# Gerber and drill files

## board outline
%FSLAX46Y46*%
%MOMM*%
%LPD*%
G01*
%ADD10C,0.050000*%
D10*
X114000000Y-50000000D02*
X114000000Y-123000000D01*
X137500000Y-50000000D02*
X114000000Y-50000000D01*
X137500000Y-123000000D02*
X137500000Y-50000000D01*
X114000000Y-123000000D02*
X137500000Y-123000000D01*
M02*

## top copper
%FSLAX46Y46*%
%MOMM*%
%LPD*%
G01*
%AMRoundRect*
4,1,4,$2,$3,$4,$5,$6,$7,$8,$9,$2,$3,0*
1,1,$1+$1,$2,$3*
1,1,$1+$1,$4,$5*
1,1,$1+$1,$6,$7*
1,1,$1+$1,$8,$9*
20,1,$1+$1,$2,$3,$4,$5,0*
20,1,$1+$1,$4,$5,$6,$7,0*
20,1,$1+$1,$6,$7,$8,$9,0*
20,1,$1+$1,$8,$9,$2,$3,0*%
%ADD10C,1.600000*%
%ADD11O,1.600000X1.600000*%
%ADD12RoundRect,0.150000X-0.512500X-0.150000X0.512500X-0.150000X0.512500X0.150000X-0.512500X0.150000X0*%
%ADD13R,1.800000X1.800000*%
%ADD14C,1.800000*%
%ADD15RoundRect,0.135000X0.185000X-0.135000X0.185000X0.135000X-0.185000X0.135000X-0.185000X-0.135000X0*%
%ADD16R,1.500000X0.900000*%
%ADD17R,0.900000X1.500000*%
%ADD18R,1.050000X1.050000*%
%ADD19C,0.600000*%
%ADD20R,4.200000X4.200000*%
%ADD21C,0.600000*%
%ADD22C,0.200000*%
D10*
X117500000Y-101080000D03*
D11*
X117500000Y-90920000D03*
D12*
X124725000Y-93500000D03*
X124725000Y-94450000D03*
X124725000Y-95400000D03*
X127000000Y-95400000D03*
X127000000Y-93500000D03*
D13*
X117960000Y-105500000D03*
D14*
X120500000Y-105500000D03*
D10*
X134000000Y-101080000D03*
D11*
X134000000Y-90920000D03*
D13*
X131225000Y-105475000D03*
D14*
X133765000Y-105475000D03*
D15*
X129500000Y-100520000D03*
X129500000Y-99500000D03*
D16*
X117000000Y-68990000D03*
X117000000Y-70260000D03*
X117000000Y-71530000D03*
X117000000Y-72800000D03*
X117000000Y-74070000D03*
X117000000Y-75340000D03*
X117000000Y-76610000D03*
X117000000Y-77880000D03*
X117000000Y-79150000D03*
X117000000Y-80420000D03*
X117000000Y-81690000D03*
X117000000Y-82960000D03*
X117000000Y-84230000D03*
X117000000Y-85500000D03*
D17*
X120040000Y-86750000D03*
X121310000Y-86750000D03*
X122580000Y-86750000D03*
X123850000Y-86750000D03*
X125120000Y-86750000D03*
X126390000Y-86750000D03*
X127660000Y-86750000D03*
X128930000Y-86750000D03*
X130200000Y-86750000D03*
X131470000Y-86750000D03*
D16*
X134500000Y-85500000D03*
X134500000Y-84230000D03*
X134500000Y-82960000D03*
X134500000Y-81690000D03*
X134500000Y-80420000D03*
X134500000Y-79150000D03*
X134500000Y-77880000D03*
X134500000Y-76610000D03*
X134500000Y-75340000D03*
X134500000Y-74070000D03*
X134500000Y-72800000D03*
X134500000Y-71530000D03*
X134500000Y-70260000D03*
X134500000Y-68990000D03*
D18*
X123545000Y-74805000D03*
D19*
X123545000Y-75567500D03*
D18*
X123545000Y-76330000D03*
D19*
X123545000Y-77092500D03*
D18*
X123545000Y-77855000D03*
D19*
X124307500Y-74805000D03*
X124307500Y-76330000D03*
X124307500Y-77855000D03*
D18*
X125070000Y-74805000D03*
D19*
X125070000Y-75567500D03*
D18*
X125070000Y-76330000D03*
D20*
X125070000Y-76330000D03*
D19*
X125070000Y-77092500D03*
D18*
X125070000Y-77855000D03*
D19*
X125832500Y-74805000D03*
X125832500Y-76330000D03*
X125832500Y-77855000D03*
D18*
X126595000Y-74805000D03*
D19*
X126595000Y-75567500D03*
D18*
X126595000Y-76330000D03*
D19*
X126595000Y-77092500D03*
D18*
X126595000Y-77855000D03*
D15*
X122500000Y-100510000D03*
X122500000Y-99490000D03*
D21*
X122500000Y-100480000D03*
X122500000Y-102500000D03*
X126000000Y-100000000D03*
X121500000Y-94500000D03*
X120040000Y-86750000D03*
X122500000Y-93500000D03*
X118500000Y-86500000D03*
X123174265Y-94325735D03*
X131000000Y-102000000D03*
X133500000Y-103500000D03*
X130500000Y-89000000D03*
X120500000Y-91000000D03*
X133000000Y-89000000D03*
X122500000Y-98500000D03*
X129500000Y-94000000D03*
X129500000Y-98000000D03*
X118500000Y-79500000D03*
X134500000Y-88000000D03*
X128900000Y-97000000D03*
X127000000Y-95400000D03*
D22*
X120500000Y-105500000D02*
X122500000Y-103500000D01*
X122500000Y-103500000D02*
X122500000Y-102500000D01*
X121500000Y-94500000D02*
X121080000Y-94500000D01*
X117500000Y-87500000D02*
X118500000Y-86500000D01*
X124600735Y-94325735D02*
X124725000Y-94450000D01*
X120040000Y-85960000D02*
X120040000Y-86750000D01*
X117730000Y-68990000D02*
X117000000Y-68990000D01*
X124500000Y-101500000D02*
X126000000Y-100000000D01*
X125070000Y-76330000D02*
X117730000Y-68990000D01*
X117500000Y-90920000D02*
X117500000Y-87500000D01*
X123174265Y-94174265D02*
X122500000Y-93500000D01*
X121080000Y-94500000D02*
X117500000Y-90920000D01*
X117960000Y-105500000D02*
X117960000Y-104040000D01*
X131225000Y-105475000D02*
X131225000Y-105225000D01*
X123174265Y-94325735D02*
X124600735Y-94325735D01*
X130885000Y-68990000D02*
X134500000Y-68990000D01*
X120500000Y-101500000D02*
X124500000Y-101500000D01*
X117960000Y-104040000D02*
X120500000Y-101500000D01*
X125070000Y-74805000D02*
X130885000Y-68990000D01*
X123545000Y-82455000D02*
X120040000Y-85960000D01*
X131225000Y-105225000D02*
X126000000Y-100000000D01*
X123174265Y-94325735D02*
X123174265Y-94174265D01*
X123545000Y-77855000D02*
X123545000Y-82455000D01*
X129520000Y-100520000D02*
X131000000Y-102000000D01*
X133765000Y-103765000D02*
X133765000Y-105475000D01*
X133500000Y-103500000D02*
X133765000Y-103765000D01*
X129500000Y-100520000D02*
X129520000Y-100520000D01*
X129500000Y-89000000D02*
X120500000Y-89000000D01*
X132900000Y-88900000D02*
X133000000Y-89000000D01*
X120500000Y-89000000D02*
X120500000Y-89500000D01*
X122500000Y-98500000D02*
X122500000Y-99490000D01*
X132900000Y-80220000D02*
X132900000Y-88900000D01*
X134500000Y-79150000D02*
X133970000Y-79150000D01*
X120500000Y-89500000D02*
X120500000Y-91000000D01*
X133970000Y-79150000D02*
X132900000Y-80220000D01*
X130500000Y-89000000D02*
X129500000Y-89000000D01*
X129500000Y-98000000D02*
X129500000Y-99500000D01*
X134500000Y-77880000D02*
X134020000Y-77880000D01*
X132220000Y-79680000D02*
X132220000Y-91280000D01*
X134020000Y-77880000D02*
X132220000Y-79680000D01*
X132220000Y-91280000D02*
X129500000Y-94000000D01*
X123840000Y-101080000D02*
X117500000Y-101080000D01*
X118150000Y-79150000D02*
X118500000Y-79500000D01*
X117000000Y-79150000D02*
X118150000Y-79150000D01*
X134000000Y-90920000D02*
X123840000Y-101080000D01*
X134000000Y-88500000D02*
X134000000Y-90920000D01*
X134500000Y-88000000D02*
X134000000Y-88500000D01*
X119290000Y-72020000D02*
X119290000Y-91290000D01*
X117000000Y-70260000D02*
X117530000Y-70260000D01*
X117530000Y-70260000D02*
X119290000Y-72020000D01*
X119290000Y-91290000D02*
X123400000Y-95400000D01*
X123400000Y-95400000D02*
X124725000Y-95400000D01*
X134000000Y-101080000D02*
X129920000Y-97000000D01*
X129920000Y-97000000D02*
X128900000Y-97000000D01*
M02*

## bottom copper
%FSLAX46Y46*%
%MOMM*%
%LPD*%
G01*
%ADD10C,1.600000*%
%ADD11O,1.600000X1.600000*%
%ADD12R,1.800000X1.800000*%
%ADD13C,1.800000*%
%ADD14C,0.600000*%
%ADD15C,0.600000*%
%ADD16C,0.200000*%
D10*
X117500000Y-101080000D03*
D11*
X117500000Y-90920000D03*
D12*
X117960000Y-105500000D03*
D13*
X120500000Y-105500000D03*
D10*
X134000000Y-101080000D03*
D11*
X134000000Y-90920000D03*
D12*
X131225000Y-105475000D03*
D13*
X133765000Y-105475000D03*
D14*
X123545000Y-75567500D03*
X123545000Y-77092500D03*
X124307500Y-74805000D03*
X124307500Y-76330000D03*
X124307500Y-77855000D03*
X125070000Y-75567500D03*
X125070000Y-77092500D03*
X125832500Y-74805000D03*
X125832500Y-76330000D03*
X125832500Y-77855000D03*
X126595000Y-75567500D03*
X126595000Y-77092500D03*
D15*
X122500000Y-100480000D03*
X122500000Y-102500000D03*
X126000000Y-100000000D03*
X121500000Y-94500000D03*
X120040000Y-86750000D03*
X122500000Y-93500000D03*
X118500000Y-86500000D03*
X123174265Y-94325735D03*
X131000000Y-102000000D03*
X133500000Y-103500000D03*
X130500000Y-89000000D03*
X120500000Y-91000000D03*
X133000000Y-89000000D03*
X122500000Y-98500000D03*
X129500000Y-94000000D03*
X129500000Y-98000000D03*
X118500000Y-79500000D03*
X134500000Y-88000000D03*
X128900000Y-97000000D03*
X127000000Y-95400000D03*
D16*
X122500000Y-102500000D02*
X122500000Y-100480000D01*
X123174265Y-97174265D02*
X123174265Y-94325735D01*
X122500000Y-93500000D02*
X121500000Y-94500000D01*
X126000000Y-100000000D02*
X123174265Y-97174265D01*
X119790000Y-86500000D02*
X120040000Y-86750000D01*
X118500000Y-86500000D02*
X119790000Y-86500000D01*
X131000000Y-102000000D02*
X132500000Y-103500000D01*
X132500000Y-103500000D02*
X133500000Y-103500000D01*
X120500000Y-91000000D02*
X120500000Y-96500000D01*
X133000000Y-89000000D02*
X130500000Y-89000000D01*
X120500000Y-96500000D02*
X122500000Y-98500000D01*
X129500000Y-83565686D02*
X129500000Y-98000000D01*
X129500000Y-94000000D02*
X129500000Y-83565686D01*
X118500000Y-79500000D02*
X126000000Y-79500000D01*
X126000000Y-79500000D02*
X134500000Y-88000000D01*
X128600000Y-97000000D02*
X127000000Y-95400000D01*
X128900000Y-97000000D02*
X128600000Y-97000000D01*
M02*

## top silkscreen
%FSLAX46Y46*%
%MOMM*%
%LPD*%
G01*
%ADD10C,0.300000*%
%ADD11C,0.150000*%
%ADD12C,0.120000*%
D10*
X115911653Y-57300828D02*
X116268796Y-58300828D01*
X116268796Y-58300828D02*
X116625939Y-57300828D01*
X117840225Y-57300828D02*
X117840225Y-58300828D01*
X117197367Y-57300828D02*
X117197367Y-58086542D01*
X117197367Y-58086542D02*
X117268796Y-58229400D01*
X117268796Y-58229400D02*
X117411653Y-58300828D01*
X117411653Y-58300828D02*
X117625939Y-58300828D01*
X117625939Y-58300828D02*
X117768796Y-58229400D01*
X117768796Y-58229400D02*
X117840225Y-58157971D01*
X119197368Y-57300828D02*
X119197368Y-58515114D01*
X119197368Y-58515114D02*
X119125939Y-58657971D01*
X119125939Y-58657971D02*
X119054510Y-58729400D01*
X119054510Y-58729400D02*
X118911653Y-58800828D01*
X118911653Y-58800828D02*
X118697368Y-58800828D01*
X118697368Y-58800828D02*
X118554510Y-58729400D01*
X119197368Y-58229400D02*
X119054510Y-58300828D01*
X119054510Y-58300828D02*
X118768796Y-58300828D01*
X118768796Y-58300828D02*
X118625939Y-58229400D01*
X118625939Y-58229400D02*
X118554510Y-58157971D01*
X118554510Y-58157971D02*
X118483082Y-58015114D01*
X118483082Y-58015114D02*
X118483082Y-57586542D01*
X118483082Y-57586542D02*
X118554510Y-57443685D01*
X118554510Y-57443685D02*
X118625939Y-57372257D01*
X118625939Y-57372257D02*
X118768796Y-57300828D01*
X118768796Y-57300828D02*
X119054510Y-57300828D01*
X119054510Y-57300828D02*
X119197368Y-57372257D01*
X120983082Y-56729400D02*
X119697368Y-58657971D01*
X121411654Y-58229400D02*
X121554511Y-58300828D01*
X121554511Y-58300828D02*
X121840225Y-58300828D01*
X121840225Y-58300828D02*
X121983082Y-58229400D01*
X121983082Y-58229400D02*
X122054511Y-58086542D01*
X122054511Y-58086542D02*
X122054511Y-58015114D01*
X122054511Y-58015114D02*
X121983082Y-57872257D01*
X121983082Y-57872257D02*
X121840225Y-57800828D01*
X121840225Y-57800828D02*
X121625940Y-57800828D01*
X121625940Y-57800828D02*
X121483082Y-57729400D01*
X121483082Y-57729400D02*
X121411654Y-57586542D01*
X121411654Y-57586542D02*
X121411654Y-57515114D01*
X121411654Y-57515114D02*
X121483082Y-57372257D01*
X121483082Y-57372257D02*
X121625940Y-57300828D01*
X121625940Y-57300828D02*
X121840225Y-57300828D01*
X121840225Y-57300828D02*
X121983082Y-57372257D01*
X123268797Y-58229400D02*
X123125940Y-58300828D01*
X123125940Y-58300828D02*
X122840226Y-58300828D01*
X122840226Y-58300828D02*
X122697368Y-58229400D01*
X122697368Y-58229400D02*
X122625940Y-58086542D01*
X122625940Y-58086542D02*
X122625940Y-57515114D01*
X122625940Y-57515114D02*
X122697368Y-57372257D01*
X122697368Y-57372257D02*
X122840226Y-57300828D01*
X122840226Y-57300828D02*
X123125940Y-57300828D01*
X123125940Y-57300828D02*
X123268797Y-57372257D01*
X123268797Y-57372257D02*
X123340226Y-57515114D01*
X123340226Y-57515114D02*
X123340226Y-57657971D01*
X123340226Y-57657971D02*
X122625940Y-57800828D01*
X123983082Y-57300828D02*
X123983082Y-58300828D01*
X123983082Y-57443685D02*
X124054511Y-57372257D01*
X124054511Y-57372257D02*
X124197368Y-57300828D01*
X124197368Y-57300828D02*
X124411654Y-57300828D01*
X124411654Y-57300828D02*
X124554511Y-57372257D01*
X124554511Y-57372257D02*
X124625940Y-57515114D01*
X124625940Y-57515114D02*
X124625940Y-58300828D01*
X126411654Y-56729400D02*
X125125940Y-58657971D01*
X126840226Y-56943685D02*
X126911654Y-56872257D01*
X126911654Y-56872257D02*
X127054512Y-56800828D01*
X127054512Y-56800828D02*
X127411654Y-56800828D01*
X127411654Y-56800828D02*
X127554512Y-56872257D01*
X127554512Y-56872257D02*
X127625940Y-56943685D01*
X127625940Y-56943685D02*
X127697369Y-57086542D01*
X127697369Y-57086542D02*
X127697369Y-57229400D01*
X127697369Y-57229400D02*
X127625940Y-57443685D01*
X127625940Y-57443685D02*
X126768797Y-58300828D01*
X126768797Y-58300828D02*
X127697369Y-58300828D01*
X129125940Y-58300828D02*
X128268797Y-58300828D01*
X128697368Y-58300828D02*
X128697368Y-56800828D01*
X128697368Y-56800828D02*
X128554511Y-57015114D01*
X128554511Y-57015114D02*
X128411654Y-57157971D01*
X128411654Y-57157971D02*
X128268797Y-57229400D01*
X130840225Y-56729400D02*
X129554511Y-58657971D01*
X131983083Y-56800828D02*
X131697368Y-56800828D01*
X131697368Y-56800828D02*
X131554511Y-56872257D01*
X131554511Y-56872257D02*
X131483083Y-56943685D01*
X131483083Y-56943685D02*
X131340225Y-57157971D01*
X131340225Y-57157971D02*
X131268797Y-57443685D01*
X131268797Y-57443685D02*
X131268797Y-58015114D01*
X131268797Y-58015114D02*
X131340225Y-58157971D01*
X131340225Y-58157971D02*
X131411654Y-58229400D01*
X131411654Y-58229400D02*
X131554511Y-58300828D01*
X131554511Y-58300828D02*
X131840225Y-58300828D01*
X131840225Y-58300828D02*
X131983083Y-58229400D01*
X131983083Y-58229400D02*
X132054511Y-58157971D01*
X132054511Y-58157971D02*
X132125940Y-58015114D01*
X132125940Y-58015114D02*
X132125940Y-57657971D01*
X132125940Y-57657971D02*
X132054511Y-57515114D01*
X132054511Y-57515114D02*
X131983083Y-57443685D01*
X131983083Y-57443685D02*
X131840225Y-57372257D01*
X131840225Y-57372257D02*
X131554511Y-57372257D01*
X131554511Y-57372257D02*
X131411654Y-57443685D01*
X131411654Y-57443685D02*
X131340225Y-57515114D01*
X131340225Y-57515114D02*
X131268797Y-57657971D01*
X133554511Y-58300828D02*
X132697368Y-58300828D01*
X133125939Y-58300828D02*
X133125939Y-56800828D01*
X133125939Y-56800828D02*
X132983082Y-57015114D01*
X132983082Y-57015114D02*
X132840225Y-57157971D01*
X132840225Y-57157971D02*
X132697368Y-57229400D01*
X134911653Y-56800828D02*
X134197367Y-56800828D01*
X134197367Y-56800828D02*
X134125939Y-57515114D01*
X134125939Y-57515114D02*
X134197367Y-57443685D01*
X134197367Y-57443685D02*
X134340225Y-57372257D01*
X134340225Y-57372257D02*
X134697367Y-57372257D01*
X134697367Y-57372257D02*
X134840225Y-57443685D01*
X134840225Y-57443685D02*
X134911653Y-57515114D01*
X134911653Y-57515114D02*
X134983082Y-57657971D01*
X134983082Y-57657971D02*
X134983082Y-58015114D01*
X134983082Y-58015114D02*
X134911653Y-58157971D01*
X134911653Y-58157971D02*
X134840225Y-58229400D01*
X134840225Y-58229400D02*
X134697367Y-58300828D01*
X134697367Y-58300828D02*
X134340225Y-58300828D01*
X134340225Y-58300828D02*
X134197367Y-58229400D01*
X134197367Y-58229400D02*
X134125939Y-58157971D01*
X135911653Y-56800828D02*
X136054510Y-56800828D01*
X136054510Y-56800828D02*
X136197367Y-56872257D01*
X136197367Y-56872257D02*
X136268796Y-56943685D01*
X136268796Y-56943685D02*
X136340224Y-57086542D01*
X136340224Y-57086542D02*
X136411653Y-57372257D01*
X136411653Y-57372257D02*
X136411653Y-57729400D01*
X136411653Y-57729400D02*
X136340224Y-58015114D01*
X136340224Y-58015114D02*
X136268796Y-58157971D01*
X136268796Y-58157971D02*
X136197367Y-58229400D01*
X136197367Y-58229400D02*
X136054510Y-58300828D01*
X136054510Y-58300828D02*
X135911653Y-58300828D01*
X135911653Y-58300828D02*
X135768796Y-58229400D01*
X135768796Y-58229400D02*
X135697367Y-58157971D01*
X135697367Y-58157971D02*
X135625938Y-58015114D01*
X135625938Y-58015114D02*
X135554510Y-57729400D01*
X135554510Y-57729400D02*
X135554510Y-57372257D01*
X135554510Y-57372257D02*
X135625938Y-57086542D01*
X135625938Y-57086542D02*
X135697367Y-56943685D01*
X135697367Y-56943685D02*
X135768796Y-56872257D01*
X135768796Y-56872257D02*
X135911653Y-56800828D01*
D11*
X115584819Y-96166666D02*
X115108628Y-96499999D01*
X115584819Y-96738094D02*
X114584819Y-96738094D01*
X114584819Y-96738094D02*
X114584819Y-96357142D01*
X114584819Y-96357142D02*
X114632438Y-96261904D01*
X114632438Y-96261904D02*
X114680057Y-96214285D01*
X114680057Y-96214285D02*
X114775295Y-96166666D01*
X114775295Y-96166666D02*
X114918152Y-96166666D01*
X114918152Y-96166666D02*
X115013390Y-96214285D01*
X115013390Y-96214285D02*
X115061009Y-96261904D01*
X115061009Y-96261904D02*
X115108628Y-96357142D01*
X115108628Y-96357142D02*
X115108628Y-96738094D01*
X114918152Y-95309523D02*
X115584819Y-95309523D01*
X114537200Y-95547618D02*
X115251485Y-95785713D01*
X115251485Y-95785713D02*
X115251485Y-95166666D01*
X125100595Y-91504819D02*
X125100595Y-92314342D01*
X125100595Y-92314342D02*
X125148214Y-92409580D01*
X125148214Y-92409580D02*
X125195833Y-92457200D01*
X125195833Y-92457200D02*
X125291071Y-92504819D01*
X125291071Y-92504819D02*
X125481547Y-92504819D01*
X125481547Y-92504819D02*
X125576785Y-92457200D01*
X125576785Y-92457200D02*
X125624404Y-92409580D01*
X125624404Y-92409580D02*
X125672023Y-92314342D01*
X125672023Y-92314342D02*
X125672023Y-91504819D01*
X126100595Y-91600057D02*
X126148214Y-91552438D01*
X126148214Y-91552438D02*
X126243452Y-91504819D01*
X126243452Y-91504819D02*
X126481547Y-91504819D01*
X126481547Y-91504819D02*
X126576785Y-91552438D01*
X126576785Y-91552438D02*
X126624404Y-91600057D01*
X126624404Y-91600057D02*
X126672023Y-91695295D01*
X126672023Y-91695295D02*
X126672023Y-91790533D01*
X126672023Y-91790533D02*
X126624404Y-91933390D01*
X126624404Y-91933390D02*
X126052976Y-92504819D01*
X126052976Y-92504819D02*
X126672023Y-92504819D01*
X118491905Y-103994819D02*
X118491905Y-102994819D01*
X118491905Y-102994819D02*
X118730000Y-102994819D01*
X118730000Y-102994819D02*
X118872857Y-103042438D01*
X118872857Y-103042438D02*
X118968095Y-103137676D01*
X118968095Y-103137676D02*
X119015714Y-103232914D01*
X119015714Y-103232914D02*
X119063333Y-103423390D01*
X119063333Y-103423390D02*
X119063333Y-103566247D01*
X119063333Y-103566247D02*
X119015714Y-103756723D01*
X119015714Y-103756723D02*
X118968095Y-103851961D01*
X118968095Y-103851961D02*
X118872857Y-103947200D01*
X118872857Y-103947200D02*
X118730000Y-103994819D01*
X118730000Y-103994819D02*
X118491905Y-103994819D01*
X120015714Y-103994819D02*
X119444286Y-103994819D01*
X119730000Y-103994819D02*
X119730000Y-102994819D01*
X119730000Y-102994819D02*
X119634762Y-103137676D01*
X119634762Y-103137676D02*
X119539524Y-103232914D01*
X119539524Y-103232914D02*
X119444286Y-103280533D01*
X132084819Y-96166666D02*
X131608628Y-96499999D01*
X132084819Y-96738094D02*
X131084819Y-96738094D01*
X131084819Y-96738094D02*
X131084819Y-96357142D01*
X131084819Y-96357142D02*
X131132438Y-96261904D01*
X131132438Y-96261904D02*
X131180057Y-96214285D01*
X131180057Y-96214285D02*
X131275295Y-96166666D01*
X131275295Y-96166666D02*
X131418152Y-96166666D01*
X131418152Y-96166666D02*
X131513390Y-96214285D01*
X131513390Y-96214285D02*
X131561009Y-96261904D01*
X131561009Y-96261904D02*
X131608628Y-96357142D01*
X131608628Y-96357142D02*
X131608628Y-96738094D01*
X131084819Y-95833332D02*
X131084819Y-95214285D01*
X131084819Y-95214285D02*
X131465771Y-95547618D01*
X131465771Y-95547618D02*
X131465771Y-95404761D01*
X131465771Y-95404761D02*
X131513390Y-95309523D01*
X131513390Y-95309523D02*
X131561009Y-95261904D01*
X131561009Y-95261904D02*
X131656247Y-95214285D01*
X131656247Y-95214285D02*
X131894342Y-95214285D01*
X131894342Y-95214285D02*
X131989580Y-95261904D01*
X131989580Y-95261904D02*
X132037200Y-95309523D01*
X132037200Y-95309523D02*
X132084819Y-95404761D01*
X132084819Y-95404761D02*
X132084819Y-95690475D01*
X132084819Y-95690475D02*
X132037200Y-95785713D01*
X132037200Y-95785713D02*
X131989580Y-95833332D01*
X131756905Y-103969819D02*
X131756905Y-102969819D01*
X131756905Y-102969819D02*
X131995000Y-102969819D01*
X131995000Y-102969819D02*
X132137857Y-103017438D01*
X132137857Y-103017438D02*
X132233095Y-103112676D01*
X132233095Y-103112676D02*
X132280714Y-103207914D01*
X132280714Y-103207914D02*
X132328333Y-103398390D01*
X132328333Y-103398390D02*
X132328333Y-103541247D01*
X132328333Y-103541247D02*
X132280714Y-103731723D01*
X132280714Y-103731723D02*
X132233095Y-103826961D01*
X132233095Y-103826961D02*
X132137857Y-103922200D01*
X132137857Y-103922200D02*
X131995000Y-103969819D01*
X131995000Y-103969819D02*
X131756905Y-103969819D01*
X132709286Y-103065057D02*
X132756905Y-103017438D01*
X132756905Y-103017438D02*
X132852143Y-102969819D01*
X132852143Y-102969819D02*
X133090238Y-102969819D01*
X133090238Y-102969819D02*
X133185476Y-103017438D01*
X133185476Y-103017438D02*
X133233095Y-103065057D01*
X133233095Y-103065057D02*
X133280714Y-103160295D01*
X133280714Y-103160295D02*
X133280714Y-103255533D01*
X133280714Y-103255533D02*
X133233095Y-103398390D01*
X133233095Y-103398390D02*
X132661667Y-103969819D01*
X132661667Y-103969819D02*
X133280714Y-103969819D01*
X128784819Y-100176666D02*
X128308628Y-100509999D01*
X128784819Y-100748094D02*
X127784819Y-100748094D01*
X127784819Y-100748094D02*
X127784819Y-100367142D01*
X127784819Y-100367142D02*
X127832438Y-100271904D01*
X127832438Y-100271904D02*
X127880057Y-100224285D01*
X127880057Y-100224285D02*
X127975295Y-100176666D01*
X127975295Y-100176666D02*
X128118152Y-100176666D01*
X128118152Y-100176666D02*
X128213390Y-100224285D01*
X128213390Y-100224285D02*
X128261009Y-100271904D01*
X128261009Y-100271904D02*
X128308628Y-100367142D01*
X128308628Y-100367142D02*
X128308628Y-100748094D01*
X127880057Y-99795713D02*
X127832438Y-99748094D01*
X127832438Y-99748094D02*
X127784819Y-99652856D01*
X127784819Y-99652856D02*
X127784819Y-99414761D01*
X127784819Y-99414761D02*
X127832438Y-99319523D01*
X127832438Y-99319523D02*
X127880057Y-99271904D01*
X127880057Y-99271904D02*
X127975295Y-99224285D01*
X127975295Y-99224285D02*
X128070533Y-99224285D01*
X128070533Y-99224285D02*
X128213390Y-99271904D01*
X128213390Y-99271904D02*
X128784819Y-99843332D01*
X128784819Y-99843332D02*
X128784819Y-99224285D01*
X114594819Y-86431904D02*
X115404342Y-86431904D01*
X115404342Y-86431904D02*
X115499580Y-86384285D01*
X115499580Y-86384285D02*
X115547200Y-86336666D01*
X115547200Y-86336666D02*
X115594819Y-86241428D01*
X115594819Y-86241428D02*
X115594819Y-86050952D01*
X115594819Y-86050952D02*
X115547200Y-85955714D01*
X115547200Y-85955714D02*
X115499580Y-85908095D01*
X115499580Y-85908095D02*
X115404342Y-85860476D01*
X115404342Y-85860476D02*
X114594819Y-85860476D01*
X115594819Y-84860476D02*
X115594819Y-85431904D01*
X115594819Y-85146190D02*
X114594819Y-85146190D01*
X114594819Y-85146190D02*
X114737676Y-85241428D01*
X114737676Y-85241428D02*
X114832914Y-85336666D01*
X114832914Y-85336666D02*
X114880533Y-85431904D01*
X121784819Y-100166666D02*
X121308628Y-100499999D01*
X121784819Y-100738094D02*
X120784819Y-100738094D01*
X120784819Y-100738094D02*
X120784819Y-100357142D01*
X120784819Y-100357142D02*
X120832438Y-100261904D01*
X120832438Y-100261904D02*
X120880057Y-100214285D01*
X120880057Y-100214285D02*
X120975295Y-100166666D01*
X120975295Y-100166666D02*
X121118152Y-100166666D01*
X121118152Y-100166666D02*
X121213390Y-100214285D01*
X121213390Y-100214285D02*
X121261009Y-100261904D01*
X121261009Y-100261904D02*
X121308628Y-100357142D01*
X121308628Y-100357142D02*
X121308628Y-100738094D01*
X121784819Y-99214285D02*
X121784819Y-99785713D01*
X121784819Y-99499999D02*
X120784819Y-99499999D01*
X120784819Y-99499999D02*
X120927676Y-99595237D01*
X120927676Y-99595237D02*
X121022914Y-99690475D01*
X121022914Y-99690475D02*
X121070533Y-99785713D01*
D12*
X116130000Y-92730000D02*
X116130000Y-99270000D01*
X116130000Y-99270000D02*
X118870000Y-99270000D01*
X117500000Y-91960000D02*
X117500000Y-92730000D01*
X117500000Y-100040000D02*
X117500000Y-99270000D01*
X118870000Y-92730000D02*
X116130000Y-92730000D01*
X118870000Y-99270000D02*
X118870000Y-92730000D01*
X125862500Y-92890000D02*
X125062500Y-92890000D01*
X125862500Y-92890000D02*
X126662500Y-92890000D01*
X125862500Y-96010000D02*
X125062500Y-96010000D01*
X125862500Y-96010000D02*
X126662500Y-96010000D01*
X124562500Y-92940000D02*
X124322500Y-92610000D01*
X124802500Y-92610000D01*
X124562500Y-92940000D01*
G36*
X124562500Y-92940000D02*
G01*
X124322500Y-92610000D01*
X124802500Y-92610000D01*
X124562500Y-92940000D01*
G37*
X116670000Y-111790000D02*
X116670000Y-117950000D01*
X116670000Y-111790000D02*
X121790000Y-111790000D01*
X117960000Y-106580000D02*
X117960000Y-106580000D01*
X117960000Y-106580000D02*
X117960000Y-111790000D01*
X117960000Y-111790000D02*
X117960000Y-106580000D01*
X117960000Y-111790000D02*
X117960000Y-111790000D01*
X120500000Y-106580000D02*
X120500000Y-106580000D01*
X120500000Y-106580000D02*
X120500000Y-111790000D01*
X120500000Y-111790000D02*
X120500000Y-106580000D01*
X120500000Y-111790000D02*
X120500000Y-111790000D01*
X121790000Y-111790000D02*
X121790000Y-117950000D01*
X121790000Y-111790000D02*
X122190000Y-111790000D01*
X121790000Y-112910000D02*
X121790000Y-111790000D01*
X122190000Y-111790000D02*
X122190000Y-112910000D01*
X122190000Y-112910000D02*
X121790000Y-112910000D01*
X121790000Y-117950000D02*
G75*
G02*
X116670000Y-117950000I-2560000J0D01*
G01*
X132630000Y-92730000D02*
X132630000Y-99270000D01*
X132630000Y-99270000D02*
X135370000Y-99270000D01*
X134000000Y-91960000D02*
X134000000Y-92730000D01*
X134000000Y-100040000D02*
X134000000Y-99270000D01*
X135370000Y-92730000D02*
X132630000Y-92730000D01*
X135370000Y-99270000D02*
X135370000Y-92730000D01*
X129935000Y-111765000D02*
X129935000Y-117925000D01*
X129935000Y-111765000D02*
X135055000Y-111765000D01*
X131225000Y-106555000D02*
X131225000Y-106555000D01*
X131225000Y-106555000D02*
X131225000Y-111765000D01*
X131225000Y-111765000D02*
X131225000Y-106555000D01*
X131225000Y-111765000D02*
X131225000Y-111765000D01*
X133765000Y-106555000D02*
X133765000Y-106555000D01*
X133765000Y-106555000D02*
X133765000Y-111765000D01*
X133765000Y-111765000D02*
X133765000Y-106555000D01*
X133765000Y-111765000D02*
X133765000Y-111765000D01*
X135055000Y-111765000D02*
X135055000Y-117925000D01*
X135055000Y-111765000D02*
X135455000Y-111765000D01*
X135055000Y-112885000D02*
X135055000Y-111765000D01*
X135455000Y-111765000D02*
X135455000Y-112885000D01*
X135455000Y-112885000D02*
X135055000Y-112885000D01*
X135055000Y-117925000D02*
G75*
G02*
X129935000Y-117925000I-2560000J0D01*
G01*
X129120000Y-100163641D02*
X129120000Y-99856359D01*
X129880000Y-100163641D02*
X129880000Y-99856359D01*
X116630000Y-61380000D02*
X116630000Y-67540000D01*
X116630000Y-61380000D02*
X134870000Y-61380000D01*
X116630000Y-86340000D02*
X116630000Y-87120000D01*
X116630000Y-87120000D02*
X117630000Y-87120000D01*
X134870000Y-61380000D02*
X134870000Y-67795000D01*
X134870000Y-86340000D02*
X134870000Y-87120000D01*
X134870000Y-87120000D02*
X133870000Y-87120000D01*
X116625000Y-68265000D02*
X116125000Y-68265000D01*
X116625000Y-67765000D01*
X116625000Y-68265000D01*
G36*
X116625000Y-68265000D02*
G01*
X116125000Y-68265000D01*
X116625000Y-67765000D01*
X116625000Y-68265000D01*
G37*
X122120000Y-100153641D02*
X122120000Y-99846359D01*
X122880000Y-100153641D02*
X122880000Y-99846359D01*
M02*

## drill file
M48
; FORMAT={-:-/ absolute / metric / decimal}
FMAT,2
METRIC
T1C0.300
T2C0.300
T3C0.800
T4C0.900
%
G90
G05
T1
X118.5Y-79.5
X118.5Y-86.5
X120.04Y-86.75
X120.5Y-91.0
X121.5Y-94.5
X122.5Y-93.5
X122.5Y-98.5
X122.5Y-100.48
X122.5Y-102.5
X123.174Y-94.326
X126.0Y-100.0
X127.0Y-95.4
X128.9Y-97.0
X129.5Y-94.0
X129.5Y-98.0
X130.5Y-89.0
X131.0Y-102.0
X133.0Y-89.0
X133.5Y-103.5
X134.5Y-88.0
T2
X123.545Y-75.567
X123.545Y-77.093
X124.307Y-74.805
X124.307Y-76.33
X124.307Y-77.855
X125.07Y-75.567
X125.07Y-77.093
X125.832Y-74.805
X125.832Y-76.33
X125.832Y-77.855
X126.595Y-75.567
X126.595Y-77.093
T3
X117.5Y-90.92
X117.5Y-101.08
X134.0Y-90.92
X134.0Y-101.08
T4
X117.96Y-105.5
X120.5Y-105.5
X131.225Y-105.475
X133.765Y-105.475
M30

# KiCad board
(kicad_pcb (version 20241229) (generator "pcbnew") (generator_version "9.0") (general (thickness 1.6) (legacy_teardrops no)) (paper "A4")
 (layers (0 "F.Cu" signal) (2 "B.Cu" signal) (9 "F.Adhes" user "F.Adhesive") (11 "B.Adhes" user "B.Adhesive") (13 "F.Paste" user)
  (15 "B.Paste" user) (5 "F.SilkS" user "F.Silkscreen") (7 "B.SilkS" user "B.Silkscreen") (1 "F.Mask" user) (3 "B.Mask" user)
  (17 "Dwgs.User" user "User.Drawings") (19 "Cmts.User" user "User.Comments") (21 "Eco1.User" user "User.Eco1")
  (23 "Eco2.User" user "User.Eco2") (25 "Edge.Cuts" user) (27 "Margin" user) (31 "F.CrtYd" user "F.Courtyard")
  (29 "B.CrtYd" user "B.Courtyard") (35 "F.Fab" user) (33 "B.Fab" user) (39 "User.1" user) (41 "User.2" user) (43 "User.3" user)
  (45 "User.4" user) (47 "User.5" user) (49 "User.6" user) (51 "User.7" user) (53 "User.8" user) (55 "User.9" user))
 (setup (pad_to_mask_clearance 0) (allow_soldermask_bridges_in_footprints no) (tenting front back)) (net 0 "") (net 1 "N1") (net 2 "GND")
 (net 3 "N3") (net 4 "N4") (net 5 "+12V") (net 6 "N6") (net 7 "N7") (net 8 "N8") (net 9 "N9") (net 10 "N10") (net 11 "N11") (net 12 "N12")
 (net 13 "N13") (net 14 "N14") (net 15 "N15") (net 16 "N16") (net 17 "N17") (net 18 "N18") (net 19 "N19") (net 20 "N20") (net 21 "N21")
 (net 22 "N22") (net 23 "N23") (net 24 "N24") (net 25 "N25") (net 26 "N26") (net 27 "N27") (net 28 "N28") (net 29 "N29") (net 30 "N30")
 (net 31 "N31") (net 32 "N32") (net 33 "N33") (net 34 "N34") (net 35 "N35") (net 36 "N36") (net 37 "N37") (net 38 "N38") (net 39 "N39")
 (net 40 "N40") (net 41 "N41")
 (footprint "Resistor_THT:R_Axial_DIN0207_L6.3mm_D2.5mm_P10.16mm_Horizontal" (layer "F.Cu") (at 117.5 101.08 90)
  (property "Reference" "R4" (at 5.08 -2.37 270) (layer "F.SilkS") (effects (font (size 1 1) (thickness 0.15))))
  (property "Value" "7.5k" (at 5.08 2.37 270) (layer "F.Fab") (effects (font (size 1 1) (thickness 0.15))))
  (fp_line (start 8.35 -1.37) (end 1.81 -1.37) (stroke (width 0.12) (type solid)) (layer "F.SilkS"))
  (fp_line (start 1.81 -1.37) (end 1.81 1.37) (stroke (width 0.12) (type solid)) (layer "F.SilkS"))
  (fp_line (start 9.12 0) (end 8.35 0) (stroke (width 0.12) (type solid)) (layer "F.SilkS"))
  (fp_line (start 1.04 0) (end 1.81 0) (stroke (width 0.12) (type solid)) (layer "F.SilkS"))
  (fp_line (start 8.35 1.37) (end 8.35 -1.37) (stroke (width 0.12) (type solid)) (layer "F.SilkS"))
  (fp_line (start 1.81 1.37) (end 8.35 1.37) (stroke (width 0.12) (type solid)) (layer "F.SilkS"))
  (pad "1" thru_hole circle (at 0 0 90) (size 1.6 1.6) (drill 0.8) (layers "*.Cu" "*.Mask") (remove_unused_layers no) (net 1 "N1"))
  (pad "2" thru_hole oval (at 10.16 0 90) (size 1.6 1.6) (drill 0.8) (layers "*.Cu" "*.Mask") (remove_unused_layers no) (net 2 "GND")))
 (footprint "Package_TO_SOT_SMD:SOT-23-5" (layer "F.Cu") (at 125.8625 94.45)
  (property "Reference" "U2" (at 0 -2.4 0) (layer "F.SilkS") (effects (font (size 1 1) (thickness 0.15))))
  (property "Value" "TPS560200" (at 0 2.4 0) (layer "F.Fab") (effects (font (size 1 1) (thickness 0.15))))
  (fp_line (start 0 -1.56) (end -0.8 -1.56) (stroke (width 0.12) (type solid)) (layer "F.SilkS"))
  (fp_line (start 0 -1.56) (end 0.8 -1.56) (stroke (width 0.12) (type solid)) (layer "F.SilkS"))
  (fp_line (start 0 1.56) (end -0.8 1.56) (stroke (width 0.12) (type solid)) (layer "F.SilkS"))
  (fp_line (start 0 1.56) (end 0.8 1.56) (stroke (width 0.12) (type solid)) (layer "F.SilkS"))
  (fp_poly
   (pts (xy -1.3 -1.51) (xy -1.54 -1.84) (xy -1.06 -1.84) (xy -1.3 -1.51)) (stroke (width 0.12) (type solid)) (fill yes) (layer "F.SilkS"))
  (pad "1" smd roundrect (at -1.1375 -0.95) (size 1.325 0.6) (layers "F.Cu" "F.Mask" "F.Paste") (roundrect_rratio 0.25) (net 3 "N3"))
  (pad "2" smd roundrect (at -1.1375 0) (size 1.325 0.6) (layers "F.Cu" "F.Mask" "F.Paste") (roundrect_rratio 0.25) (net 2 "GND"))
  (pad "3" smd roundrect (at -1.1375 0.95) (size 1.325 0.6) (layers "F.Cu" "F.Mask" "F.Paste") (roundrect_rratio 0.25) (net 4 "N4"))
  (pad "4" smd roundrect (at 1.1375 0.95) (size 1.325 0.6) (layers "F.Cu" "F.Mask" "F.Paste") (roundrect_rratio 0.25) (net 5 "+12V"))
  (pad "5" smd roundrect (at 1.1375 -0.95) (size 1.325 0.6) (layers "F.Cu" "F.Mask" "F.Paste") (roundrect_rratio 0.25) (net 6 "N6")))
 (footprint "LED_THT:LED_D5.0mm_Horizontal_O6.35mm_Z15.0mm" (layer "F.Cu") (at 117.96 105.5)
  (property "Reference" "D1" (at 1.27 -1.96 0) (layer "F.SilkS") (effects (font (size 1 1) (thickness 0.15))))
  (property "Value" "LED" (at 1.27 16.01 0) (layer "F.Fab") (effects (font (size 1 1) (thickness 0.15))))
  (fp_line (start -1.29 6.29) (end -1.29 12.45) (stroke (width 0.12) (type solid)) (layer "F.SilkS"))
  (fp_line (start -1.29 6.29) (end 3.83 6.29) (stroke (width 0.12) (type solid)) (layer "F.SilkS"))
  (fp_line (start 0 1.08) (end 0 1.08) (stroke (width 0.12) (type solid)) (layer "F.SilkS"))
  (fp_line (start 0 1.08) (end 0 6.29) (stroke (width 0.12) (type solid)) (layer "F.SilkS"))
  (fp_line (start 0 6.29) (end 0 1.08) (stroke (width 0.12) (type solid)) (layer "F.SilkS"))
  (fp_line (start 0 6.29) (end 0 6.29) (stroke (width 0.12) (type solid)) (layer "F.SilkS"))
  (fp_line (start 2.54 1.08) (end 2.54 1.08) (stroke (width 0.12) (type solid)) (layer "F.SilkS"))
  (fp_line (start 2.54 1.08) (end 2.54 6.29) (stroke (width 0.12) (type solid)) (layer "F.SilkS"))
  (fp_line (start 2.54 6.29) (end 2.54 1.08) (stroke (width 0.12) (type solid)) (layer "F.SilkS"))
  (fp_line (start 2.54 6.29) (end 2.54 6.29) (stroke (width 0.12) (type solid)) (layer "F.SilkS"))
  (fp_line (start 3.83 6.29) (end 3.83 12.45) (stroke (width 0.12) (type solid)) (layer "F.SilkS"))
  (fp_line (start 3.83 6.29) (end 4.23 6.29) (stroke (width 0.12) (type solid)) (layer "F.SilkS"))
  (fp_line (start 3.83 7.41) (end 3.83 6.29) (stroke (width 0.12) (type solid)) (layer "F.SilkS"))
  (fp_line (start 4.23 6.29) (end 4.23 7.41) (stroke (width 0.12) (type solid)) (layer "F.SilkS"))
  (fp_line (start 4.23 7.41) (end 3.83 7.41) (stroke (width 0.12) (type solid)) (layer "F.SilkS"))
  (fp_arc (start 3.83 12.45) (mid 1.27 15.01) (end -1.29 12.45) (stroke (width 0.12) (type solid)) (layer "F.SilkS"))
  (pad "1" thru_hole rect (at 0 0) (size 1.8 1.8) (drill 0.9) (layers "*.Cu" "*.Mask") (remove_unused_layers no) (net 2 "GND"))
  (pad "2" thru_hole circle (at 2.54 0) (size 1.8 1.8) (drill 0.9) (layers "*.Cu" "*.Mask") (remove_unused_layers no) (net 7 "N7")))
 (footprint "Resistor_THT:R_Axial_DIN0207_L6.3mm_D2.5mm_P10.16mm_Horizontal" (layer "F.Cu") (at 134 101.08 90)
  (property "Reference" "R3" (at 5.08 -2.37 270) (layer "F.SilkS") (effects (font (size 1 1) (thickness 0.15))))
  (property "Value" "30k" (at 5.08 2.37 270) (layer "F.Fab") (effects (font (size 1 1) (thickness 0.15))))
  (fp_line (start 8.35 -1.37) (end 1.81 -1.37) (stroke (width 0.12) (type solid)) (layer "F.SilkS"))
  (fp_line (start 1.81 -1.37) (end 1.81 1.37) (stroke (width 0.12) (type solid)) (layer "F.SilkS"))
  (fp_line (start 9.12 0) (end 8.35 0) (stroke (width 0.12) (type solid)) (layer "F.SilkS"))
  (fp_line (start 1.04 0) (end 1.81 0) (stroke (width 0.12) (type solid)) (layer "F.SilkS"))
  (fp_line (start 8.35 1.37) (end 8.35 -1.37) (stroke (width 0.12) (type solid)) (layer "F.SilkS"))
  (fp_line (start 1.81 1.37) (end 8.35 1.37) (stroke (width 0.12) (type solid)) (layer "F.SilkS"))
  (pad "1" thru_hole circle (at 0 0 90) (size 1.6 1.6) (drill 0.8) (layers "*.Cu" "*.Mask") (remove_unused_layers no) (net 5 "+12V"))
  (pad "2" thru_hole oval (at 10.16 0 90) (size 1.6 1.6) (drill 0.8) (layers "*.Cu" "*.Mask") (remove_unused_layers no) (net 1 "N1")))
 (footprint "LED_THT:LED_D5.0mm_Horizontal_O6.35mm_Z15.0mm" (layer "F.Cu") (at 131.225 105.475)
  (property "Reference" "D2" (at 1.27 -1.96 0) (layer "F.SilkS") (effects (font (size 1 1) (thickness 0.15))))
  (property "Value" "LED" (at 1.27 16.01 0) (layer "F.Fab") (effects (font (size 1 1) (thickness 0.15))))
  (fp_line (start -1.29 6.29) (end -1.29 12.45) (stroke (width 0.12) (type solid)) (layer "F.SilkS"))
  (fp_line (start -1.29 6.29) (end 3.83 6.29) (stroke (width 0.12) (type solid)) (layer "F.SilkS"))
  (fp_line (start 0 1.08) (end 0 1.08) (stroke (width 0.12) (type solid)) (layer "F.SilkS"))
  (fp_line (start 0 1.08) (end 0 6.29) (stroke (width 0.12) (type solid)) (layer "F.SilkS"))
  (fp_line (start 0 6.29) (end 0 1.08) (stroke (width 0.12) (type solid)) (layer "F.SilkS"))
  (fp_line (start 0 6.29) (end 0 6.29) (stroke (width 0.12) (type solid)) (layer "F.SilkS"))
  (fp_line (start 2.54 1.08) (end 2.54 1.08) (stroke (width 0.12) (type solid)) (layer "F.SilkS"))
  (fp_line (start 2.54 1.08) (end 2.54 6.29) (stroke (width 0.12) (type solid)) (layer "F.SilkS"))
  (fp_line (start 2.54 6.29) (end 2.54 1.08) (stroke (width 0.12) (type solid)) (layer "F.SilkS"))
  (fp_line (start 2.54 6.29) (end 2.54 6.29) (stroke (width 0.12) (type solid)) (layer "F.SilkS"))
  (fp_line (start 3.83 6.29) (end 3.83 12.45) (stroke (width 0.12) (type solid)) (layer "F.SilkS"))
  (fp_line (start 3.83 6.29) (end 4.23 6.29) (stroke (width 0.12) (type solid)) (layer "F.SilkS"))
  (fp_line (start 3.83 7.41) (end 3.83 6.29) (stroke (width 0.12) (type solid)) (layer "F.SilkS"))
  (fp_line (start 4.23 6.29) (end 4.23 7.41) (stroke (width 0.12) (type solid)) (layer "F.SilkS"))
  (fp_line (start 4.23 7.41) (end 3.83 7.41) (stroke (width 0.12) (type solid)) (layer "F.SilkS"))
  (fp_arc (start 3.83 12.45) (mid 1.27 15.01) (end -1.29 12.45) (stroke (width 0.12) (type solid)) (layer "F.SilkS"))
  (pad "1" thru_hole rect (at 0 0) (size 1.8 1.8) (drill 0.9) (layers "*.Cu" "*.Mask") (remove_unused_layers no) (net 2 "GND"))
  (pad "2" thru_hole circle (at 2.54 0) (size 1.8 1.8) (drill 0.9) (layers "*.Cu" "*.Mask") (remove_unused_layers no) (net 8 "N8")))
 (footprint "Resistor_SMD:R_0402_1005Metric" (layer "F.Cu") (at 129.5 100.01 90)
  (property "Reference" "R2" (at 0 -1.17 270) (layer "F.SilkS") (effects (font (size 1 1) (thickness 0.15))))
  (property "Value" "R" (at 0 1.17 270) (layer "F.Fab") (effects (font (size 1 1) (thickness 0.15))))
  (fp_line (start -0.153641 -0.38) (end 0.153641 -0.38) (stroke (width 0.12) (type solid)) (layer "F.SilkS"))
  (fp_line (start -0.153641 0.38) (end 0.153641 0.38) (stroke (width 0.12) (type solid)) (layer "F.SilkS"))
  (pad "1" smd roundrect (at -0.51 0 90) (size 0.54 0.64) (layers "F.Cu" "F.Mask" "F.Paste") (roundrect_rratio 0.25) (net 8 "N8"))
  (pad "2" smd roundrect (at 0.51 0 90) (size 0.54 0.64) (layers "F.Cu" "F.Mask" "F.Paste") (roundrect_rratio 0.25) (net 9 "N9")))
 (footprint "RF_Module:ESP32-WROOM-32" (layer "F.Cu") (at 125.75 77.24)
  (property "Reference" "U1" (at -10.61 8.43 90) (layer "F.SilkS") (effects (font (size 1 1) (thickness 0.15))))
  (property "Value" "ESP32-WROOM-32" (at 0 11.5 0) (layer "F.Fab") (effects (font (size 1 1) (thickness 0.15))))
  (fp_line (start -9.12 -15.86) (end -9.12 -9.7) (stroke (width 0.12) (type solid)) (layer "F.SilkS"))
  (fp_line (start -9.12 -15.86) (end 9.12 -15.86) (stroke (width 0.12) (type solid)) (layer "F.SilkS"))
  (fp_line (start -9.12 9.1) (end -9.12 9.88) (stroke (width 0.12) (type solid)) (layer "F.SilkS"))
  (fp_line (start -9.12 9.88) (end -8.12 9.88) (stroke (width 0.12) (type solid)) (layer "F.SilkS"))
  (fp_line (start 9.12 -15.86) (end 9.12 -9.445) (stroke (width 0.12) (type solid)) (layer "F.SilkS"))
  (fp_line (start 9.12 9.1) (end 9.12 9.88) (stroke (width 0.12) (type solid)) (layer "F.SilkS"))
  (fp_line (start 9.12 9.88) (end 8.12 9.88) (stroke (width 0.12) (type solid)) (layer "F.SilkS"))
  (fp_poly
   (pts (xy -9.125 -8.975) (xy -9.625 -8.975) (xy -9.125 -9.475) (xy -9.125 -8.975)) (stroke (width 0.12) (type solid)) (fill yes)
   (layer "F.SilkS"))
  (pad "1" smd rect (at -8.75 -8.25) (size 1.5 0.9) (layers "F.Cu" "F.Mask" "F.Paste") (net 2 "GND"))
  (pad "2" smd rect (at -8.75 -6.98) (size 1.5 0.9) (layers "F.Cu" "F.Mask" "F.Paste") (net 4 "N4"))
  (pad "3" smd rect (at -8.75 -5.71) (size 1.5 0.9) (layers "F.Cu" "F.Mask" "F.Paste") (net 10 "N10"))
  (pad "4" smd rect (at -8.75 -4.44) (size 1.5 0.9) (layers "F.Cu" "F.Mask" "F.Paste") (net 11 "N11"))
  (pad "5" smd rect (at -8.75 -3.17) (size 1.5 0.9) (layers "F.Cu" "F.Mask" "F.Paste") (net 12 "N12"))
  (pad "6" smd rect (at -8.75 -1.9) (size 1.5 0.9) (layers "F.Cu" "F.Mask" "F.Paste") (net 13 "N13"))
  (pad "7" smd rect (at -8.75 -0.63) (size 1.5 0.9) (layers "F.Cu" "F.Mask" "F.Paste") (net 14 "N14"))
  (pad "8" smd rect (at -8.75 0.64) (size 1.5 0.9) (layers "F.Cu" "F.Mask" "F.Paste") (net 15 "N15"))
  (pad "9" smd rect (at -8.75 1.91) (size 1.5 0.9) (layers "F.Cu" "F.Mask" "F.Paste") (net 1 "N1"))
  (pad "10" smd rect (at -8.75 3.18) (size 1.5 0.9) (layers "F.Cu" "F.Mask" "F.Paste") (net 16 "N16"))
  (pad "11" smd rect (at -8.75 4.45) (size 1.5 0.9) (layers "F.Cu" "F.Mask" "F.Paste") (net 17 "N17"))
  (pad "12" smd rect (at -8.75 5.72) (size 1.5 0.9) (layers "F.Cu" "F.Mask" "F.Paste") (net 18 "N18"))
  (pad "13" smd rect (at -8.75 6.99) (size 1.5 0.9) (layers "F.Cu" "F.Mask" "F.Paste") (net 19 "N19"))
  (pad "14" smd rect (at -8.75 8.26) (size 1.5 0.9) (layers "F.Cu" "F.Mask" "F.Paste") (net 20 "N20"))
  (pad "15" smd rect (at -5.71 9.51 90) (size 1.5 0.9) (layers "F.Cu" "F.Mask" "F.Paste") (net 2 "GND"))
  (pad "16" smd rect (at -4.44 9.51 90) (size 1.5 0.9) (layers "F.Cu" "F.Mask" "F.Paste") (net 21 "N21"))
  (pad "17" smd rect (at -3.17 9.51 90) (size 1.5 0.9) (layers "F.Cu" "F.Mask" "F.Paste") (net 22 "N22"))
  (pad "18" smd rect (at -1.9 9.51 90) (size 1.5 0.9) (layers "F.Cu" "F.Mask" "F.Paste") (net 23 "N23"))
  (pad "19" smd rect (at -0.63 9.51 90) (size 1.5 0.9) (layers "F.Cu" "F.Mask" "F.Paste") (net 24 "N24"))
  (pad "20" smd rect (at 0.64 9.51 90) (size 1.5 0.9) (layers "F.Cu" "F.Mask" "F.Paste") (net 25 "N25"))
  (pad "21" smd rect (at 1.91 9.51 90) (size 1.5 0.9) (layers "F.Cu" "F.Mask" "F.Paste") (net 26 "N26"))
  (pad "22" smd rect (at 3.18 9.51 90) (size 1.5 0.9) (layers "F.Cu" "F.Mask" "F.Paste") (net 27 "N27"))
  (pad "23" smd rect (at 4.45 9.51 90) (size 1.5 0.9) (layers "F.Cu" "F.Mask" "F.Paste") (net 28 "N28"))
  (pad "24" smd rect (at 5.72 9.51 90) (size 1.5 0.9) (layers "F.Cu" "F.Mask" "F.Paste") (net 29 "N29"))
  (pad "25" smd rect (at 8.75 8.26) (size 1.5 0.9) (layers "F.Cu" "F.Mask" "F.Paste") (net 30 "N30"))
  (pad "26" smd rect (at 8.75 6.99) (size 1.5 0.9) (layers "F.Cu" "F.Mask" "F.Paste") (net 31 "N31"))
  (pad "27" smd rect (at 8.75 5.72) (size 1.5 0.9) (layers "F.Cu" "F.Mask" "F.Paste") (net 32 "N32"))
  (pad "28" smd rect (at 8.75 4.45) (size 1.5 0.9) (layers "F.Cu" "F.Mask" "F.Paste") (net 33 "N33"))
  (pad "29" smd rect (at 8.75 3.18) (size 1.5 0.9) (layers "F.Cu" "F.Mask" "F.Paste") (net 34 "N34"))
  (pad "30" smd rect (at 8.75 1.91) (size 1.5 0.9) (layers "F.Cu" "F.Mask" "F.Paste") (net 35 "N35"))
  (pad "31" smd rect (at 8.75 0.64) (size 1.5 0.9) (layers "F.Cu" "F.Mask" "F.Paste") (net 9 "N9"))
  (pad "32" smd rect (at 8.75 -0.63) (size 1.5 0.9) (layers "F.Cu" "F.Mask" "F.Paste") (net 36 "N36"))
  (pad "33" smd rect (at 8.75 -1.9) (size 1.5 0.9) (layers "F.Cu" "F.Mask" "F.Paste") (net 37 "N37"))
  (pad "34" smd rect (at 8.75 -3.17) (size 1.5 0.9) (layers "F.Cu" "F.Mask" "F.Paste") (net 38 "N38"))
  (pad "35" smd rect (at 8.75 -4.44) (size 1.5 0.9) (layers "F.Cu" "F.Mask" "F.Paste") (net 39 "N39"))
  (pad "36" smd rect (at 8.75 -5.71) (size 1.5 0.9) (layers "F.Cu" "F.Mask" "F.Paste") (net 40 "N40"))
  (pad "37" smd rect (at 8.75 -6.98) (size 1.5 0.9) (layers "F.Cu" "F.Mask" "F.Paste") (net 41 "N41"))
  (pad "38" smd rect (at 8.75 -8.25) (size 1.5 0.9) (layers "F.Cu" "F.Mask" "F.Paste") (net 2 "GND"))
  (pad "39" smd rect (at -2.205 -2.435) (size 1.05 1.05) (layers "F.Cu" "F.Paste") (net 2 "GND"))
  (pad "39" thru_hole circle (at -2.205 -1.6725) (size 0.6 0.6) (drill 0.3) (layers "*.Cu" "F.Mask") (remove_unused_layers no) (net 2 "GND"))
  (pad "39" smd rect (at -2.205 -0.91) (size 1.05 1.05) (layers "F.Cu" "F.Paste") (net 2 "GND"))
  (pad "39" thru_hole circle (at -2.205 -0.1475) (size 0.6 0.6) (drill 0.3) (layers "*.Cu" "F.Mask") (remove_unused_layers no) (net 2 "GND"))
  (pad "39" smd rect (at -2.205 0.615) (size 1.05 1.05) (layers "F.Cu" "F.Paste") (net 2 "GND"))
  (pad "39" thru_hole circle (at -1.4425 -2.435) (size 0.6 0.6) (drill 0.3) (layers "*.Cu" "F.Mask") (remove_unused_layers no) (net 2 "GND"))
  (pad "39" thru_hole circle (at -1.4425 -0.91) (size 0.6 0.6) (drill 0.3) (layers "*.Cu" "F.Mask") (remove_unused_layers no) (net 2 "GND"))
  (pad "39" thru_hole circle (at -1.4425 0.615) (size 0.6 0.6) (drill 0.3) (layers "*.Cu" "F.Mask") (remove_unused_layers no) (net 2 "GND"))
  (pad "39" smd rect (at -0.68 -2.435) (size 1.05 1.05) (layers "F.Cu" "F.Paste") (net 2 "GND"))
  (pad "39" thru_hole circle (at -0.68 -1.6725) (size 0.6 0.6) (drill 0.3) (layers "*.Cu" "F.Mask") (remove_unused_layers no) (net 2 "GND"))
  (pad "39" smd rect (at -0.68 -0.91) (size 1.05 1.05) (layers "F.Cu" "F.Paste") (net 2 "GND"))
  (pad "39" smd rect (at -0.68 -0.91) (size 4.2 4.2) (layers "F.Cu" "F.Mask") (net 2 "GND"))
  (pad "39" thru_hole circle (at -0.68 -0.1475) (size 0.6 0.6) (drill 0.3) (layers "*.Cu" "F.Mask") (remove_unused_layers no) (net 2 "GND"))
  (pad "39" smd rect (at -0.68 0.615) (size 1.05 1.05) (layers "F.Cu" "F.Paste") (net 2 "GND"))
  (pad "39" thru_hole circle (at 0.0825 -2.435) (size 0.6 0.6) (drill 0.3) (layers "*.Cu" "F.Mask") (remove_unused_layers no) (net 2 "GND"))
  (pad "39" thru_hole circle (at 0.0825 -0.91) (size 0.6 0.6) (drill 0.3) (layers "*.Cu" "F.Mask") (remove_unused_layers no) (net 2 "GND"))
  (pad "39" thru_hole circle (at 0.0825 0.615) (size 0.6 0.6) (drill 0.3) (layers "*.Cu" "F.Mask") (remove_unused_layers no) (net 2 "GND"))
  (pad "39" smd rect (at 0.845 -2.435) (size 1.05 1.05) (layers "F.Cu" "F.Paste") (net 2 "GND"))
  (pad "39" thru_hole circle (at 0.845 -1.6725) (size 0.6 0.6) (drill 0.3) (layers "*.Cu" "F.Mask" "B.SilkS") (remove_unused_layers no)
   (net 2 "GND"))
  (pad "39" smd rect (at 0.845 -0.91) (size 1.05 1.05) (layers "F.Cu" "F.Paste") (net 2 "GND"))
  (pad "39" thru_hole circle (at 0.845 -0.1475) (size 0.6 0.6) (drill 0.3) (layers "*.Cu" "F.Mask") (remove_unused_layers no) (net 2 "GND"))
  (pad "39" smd rect (at 0.845 0.615) (size 1.05 1.05) (layers "F.Cu" "F.Paste") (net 2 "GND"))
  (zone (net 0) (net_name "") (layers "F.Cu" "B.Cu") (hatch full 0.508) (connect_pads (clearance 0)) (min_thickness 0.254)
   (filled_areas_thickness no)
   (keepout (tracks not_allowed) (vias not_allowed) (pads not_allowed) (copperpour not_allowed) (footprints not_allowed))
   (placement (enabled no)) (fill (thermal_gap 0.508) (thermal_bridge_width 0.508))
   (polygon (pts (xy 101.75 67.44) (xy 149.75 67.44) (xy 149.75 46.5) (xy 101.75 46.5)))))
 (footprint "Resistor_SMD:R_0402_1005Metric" (layer "F.Cu") (at 122.5 100 90)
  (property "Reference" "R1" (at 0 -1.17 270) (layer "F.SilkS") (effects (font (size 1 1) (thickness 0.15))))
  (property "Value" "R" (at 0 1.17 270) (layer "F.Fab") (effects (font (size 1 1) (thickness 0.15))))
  (fp_line (start -0.153641 -0.38) (end 0.153641 -0.38) (stroke (width 0.12) (type solid)) (layer "F.SilkS"))
  (fp_line (start -0.153641 0.38) (end 0.153641 0.38) (stroke (width 0.12) (type solid)) (layer "F.SilkS"))
  (pad "1" smd roundrect (at -0.51 0 90) (size 0.54 0.64) (layers "F.Cu" "F.Mask" "F.Paste") (roundrect_rratio 0.25) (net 7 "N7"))
  (pad "2" smd roundrect (at 0.51 0 90) (size 0.54 0.64) (layers "F.Cu" "F.Mask" "F.Paste") (roundrect_rratio 0.25) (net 35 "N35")))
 (gr_line (start 114 50) (end 114 123) (stroke (width 0.05) (type default)) (layer "Edge.Cuts"))
 (gr_line (start 137.5 50) (end 114 50) (stroke (width 0.05) (type default)) (layer "Edge.Cuts"))
 (gr_line (start 137.5 123) (end 137.5 50) (stroke (width 0.05) (type default)) (layer "Edge.Cuts"))
 (gr_line (start 114 123) (end 137.5 123) (stroke (width 0.05) (type default)) (layer "Edge.Cuts"))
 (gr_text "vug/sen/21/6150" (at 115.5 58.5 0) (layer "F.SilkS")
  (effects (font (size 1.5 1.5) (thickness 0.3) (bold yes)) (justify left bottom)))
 (segment (start 120.5 105.5) (end 122.5 103.5) (width 0.2) (layer "F.Cu") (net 7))
 (segment (start 122.5 103.5) (end 122.5 102.5) (width 0.2) (layer "F.Cu") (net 7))
 (via (at 122.5 100.48) (size 0.6) (drill 0.3) (layers "F.Cu" "B.Cu") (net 7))
 (via (at 122.5 102.5) (size 0.6) (drill 0.3) (layers "F.Cu" "B.Cu") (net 7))
 (segment (start 122.5 102.5) (end 122.5 100.48) (width 0.2) (layer "B.Cu") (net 7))
 (segment (start 121.5 94.5) (end 121.08 94.5) (width 0.2) (layer "F.Cu") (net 2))
 (segment (start 117.5 87.5) (end 118.5 86.5) (width 0.2) (layer "F.Cu") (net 2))
 (segment (start 124.600735 94.325735) (end 124.725 94.45) (width 0.2) (layer "F.Cu") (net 2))
 (segment (start 120.04 85.96) (end 120.04 86.75) (width 0.2) (layer "F.Cu") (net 2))
 (segment (start 117.73 68.99) (end 117 68.99) (width 0.2) (layer "F.Cu") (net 2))
 (segment (start 124.5 101.5) (end 126 100) (width 0.2) (layer "F.Cu") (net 2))
 (segment (start 125.07 76.33) (end 117.73 68.99) (width 0.2) (layer "F.Cu") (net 2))
 (segment (start 117.5 90.92) (end 117.5 87.5) (width 0.2) (layer "F.Cu") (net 2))
 (segment (start 123.174265 94.174265) (end 122.5 93.5) (width 0.2) (layer "F.Cu") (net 2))
 (segment (start 121.08 94.5) (end 117.5 90.92) (width 0.2) (layer "F.Cu") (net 2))
 (segment (start 117.96 105.5) (end 117.96 104.04) (width 0.2) (layer "F.Cu") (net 2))
 (segment (start 131.225 105.475) (end 131.225 105.225) (width 0.2) (layer "F.Cu") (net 2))
 (segment (start 123.174265 94.325735) (end 124.600735 94.325735) (width 0.2) (layer "F.Cu") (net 2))
 (segment (start 130.885 68.99) (end 134.5 68.99) (width 0.2) (layer "F.Cu") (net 2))
 (segment (start 120.5 101.5) (end 124.5 101.5) (width 0.2) (layer "F.Cu") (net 2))
 (segment (start 117.96 104.04) (end 120.5 101.5) (width 0.2) (layer "F.Cu") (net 2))
 (segment (start 125.07 74.805) (end 130.885 68.99) (width 0.2) (layer "F.Cu") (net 2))
 (segment (start 123.545 82.455) (end 120.04 85.96) (width 0.2) (layer "F.Cu") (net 2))
 (segment (start 131.225 105.225) (end 126 100) (width 0.2) (layer "F.Cu") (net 2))
 (segment (start 123.174265 94.325735) (end 123.174265 94.174265) (width 0.2) (layer "F.Cu") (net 2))
 (segment (start 123.545 77.855) (end 123.545 82.455) (width 0.2) (layer "F.Cu") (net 2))
 (via (at 126 100) (size 0.6) (drill 0.3) (layers "F.Cu" "B.Cu") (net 2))
 (via (at 121.5 94.5) (size 0.6) (drill 0.3) (layers "F.Cu" "B.Cu") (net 2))
 (via (at 120.04 86.75) (size 0.6) (drill 0.3) (layers "F.Cu" "B.Cu") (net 2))
 (via (at 122.5 93.5) (size 0.6) (drill 0.3) (layers "F.Cu" "B.Cu") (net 2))
 (via (at 118.5 86.5) (size 0.6) (drill 0.3) (layers "F.Cu" "B.Cu") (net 2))
 (via (at 123.174265 94.325735) (size 0.6) (drill 0.3) (layers "F.Cu" "B.Cu") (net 2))
 (segment (start 123.174265 97.174265) (end 123.174265 94.325735) (width 0.2) (layer "B.Cu") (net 2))
 (segment (start 122.5 93.5) (end 121.5 94.5) (width 0.2) (layer "B.Cu") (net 2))
 (segment (start 126 100) (end 123.174265 97.174265) (width 0.2) (layer "B.Cu") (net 2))
 (segment (start 119.79 86.5) (end 120.04 86.75) (width 0.2) (layer "B.Cu") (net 2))
 (segment (start 118.5 86.5) (end 119.79 86.5) (width 0.2) (layer "B.Cu") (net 2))
 (segment (start 129.52 100.52) (end 131 102) (width 0.2) (layer "F.Cu") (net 8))
 (segment (start 133.765 103.765) (end 133.765 105.475) (width 0.2) (layer "F.Cu") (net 8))
 (segment (start 133.5 103.5) (end 133.765 103.765) (width 0.2) (layer "F.Cu") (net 8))
 (segment (start 129.5 100.52) (end 129.52 100.52) (width 0.2) (layer "F.Cu") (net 8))
 (via (at 131 102) (size 0.6) (drill 0.3) (layers "F.Cu" "B.Cu") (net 8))
 (via (at 133.5 103.5) (size 0.6) (drill 0.3) (layers "F.Cu" "B.Cu") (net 8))
 (segment (start 131 102) (end 132.5 103.5) (width 0.2) (layer "B.Cu") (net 8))
 (segment (start 132.5 103.5) (end 133.5 103.5) (width 0.2) (layer "B.Cu") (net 8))
 (segment (start 129.5 89) (end 120.5 89) (width 0.2) (layer "F.Cu") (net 35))
 (segment (start 132.9 88.9) (end 133 89) (width 0.2) (layer "F.Cu") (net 35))
 (segment (start 120.5 89) (end 120.5 89.5) (width 0.2) (layer "F.Cu") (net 35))
 (segment (start 122.5 98.5) (end 122.5 99.49) (width 0.2) (layer "F.Cu") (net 35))
 (segment (start 132.9 80.22) (end 132.9 88.9) (width 0.2) (layer "F.Cu") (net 35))
 (segment (start 134.5 79.15) (end 133.97 79.15) (width 0.2) (layer "F.Cu") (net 35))
 (segment (start 120.5 89.5) (end 120.5 91) (width 0.2) (layer "F.Cu") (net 35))
 (segment (start 133.97 79.15) (end 132.9 80.22) (width 0.2) (layer "F.Cu") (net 35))
 (segment (start 130.5 89) (end 129.5 89) (width 0.2) (layer "F.Cu") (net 35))
 (via (at 130.5 89) (size 0.6) (drill 0.3) (layers "F.Cu" "B.Cu") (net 35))
 (via (at 120.5 91) (size 0.6) (drill 0.3) (layers "F.Cu" "B.Cu") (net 35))
 (via (at 133 89) (size 0.6) (drill 0.3) (layers "F.Cu" "B.Cu") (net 35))
 (via (at 122.5 98.5) (size 0.6) (drill 0.3) (layers "F.Cu" "B.Cu") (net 35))
 (segment (start 120.5 91) (end 120.5 96.5) (width 0.2) (layer "B.Cu") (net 35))
 (segment (start 133 89) (end 130.5 89) (width 0.2) (layer "B.Cu") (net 35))
 (segment (start 120.5 96.5) (end 122.5 98.5) (width 0.2) (layer "B.Cu") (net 35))
 (segment (start 129.5 98) (end 129.5 99.5) (width 0.2) (layer "F.Cu") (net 9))
 (segment (start 134.5 77.88) (end 134.02 77.88) (width 0.2) (layer "F.Cu") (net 9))
 (segment (start 132.22 79.68) (end 132.22 91.28) (width 0.2) (layer "F.Cu") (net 9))
 (segment (start 134.02 77.88) (end 132.22 79.68) (width 0.2) (layer "F.Cu") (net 9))
 (segment (start 132.22 91.28) (end 129.5 94) (width 0.2) (layer "F.Cu") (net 9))
 (via (at 129.5 94) (size 0.6) (drill 0.3) (layers "F.Cu" "B.Cu") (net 9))
 (via (at 129.5 98) (size 0.6) (drill 0.3) (layers "F.Cu" "B.Cu") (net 9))
 (segment (start 129.5 83.565686) (end 129.5 98) (width 0.2) (layer "B.Cu") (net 9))
 (segment (start 129.5 94) (end 129.5 83.565686) (width 0.2) (layer "B.Cu") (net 9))
 (segment (start 123.84 101.08) (end 117.5 101.08) (width 0.2) (layer "F.Cu") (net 1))
 (segment (start 118.15 79.15) (end 118.5 79.5) (width 0.2) (layer "F.Cu") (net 1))
 (segment (start 117 79.15) (end 118.15 79.15) (width 0.2) (layer "F.Cu") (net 1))
 (segment (start 134 90.92) (end 123.84 101.08) (width 0.2) (layer "F.Cu") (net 1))
 (segment (start 134 88.5) (end 134 90.92) (width 0.2) (layer "F.Cu") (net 1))
 (segment (start 134.5 88) (end 134 88.5) (width 0.2) (layer "F.Cu") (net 1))
 (via (at 118.5 79.5) (size 0.6) (drill 0.3) (layers "F.Cu" "B.Cu") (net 1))
 (via (at 134.5 88) (size 0.6) (drill 0.3) (layers "F.Cu" "B.Cu") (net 1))
 (segment (start 118.5 79.5) (end 126 79.5) (width 0.2) (layer "B.Cu") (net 1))
 (segment (start 126 79.5) (end 134.5 88) (width 0.2) (layer "B.Cu") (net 1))
 (segment (start 119.29 72.02) (end 119.29 91.29) (width 0.2) (layer "F.Cu") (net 4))
 (segment (start 117 70.26) (end 117.53 70.26) (width 0.2) (layer "F.Cu") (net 4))
 (segment (start 117.53 70.26) (end 119.29 72.02) (width 0.2) (layer "F.Cu") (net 4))
 (segment (start 119.29 91.29) (end 123.4 95.4) (width 0.2) (layer "F.Cu") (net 4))
 (segment (start 123.4 95.4) (end 124.725 95.4) (width 0.2) (layer "F.Cu") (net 4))
 (segment (start 134 101.08) (end 129.92 97) (width 0.2) (layer "F.Cu") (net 5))
 (segment (start 129.92 97) (end 128.9 97) (width 0.2) (layer "F.Cu") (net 5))
 (via (at 128.9 97) (size 0.6) (drill 0.3) (layers "F.Cu" "B.Cu") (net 5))
 (via (at 127 95.4) (size 0.6) (drill 0.3) (layers "F.Cu" "B.Cu") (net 5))
 (segment (start 128.6 97) (end 127 95.4) (width 0.2) (layer "B.Cu") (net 5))
 (segment (start 128.9 97) (end 128.6 97) (width 0.2) (layer "B.Cu") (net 5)))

